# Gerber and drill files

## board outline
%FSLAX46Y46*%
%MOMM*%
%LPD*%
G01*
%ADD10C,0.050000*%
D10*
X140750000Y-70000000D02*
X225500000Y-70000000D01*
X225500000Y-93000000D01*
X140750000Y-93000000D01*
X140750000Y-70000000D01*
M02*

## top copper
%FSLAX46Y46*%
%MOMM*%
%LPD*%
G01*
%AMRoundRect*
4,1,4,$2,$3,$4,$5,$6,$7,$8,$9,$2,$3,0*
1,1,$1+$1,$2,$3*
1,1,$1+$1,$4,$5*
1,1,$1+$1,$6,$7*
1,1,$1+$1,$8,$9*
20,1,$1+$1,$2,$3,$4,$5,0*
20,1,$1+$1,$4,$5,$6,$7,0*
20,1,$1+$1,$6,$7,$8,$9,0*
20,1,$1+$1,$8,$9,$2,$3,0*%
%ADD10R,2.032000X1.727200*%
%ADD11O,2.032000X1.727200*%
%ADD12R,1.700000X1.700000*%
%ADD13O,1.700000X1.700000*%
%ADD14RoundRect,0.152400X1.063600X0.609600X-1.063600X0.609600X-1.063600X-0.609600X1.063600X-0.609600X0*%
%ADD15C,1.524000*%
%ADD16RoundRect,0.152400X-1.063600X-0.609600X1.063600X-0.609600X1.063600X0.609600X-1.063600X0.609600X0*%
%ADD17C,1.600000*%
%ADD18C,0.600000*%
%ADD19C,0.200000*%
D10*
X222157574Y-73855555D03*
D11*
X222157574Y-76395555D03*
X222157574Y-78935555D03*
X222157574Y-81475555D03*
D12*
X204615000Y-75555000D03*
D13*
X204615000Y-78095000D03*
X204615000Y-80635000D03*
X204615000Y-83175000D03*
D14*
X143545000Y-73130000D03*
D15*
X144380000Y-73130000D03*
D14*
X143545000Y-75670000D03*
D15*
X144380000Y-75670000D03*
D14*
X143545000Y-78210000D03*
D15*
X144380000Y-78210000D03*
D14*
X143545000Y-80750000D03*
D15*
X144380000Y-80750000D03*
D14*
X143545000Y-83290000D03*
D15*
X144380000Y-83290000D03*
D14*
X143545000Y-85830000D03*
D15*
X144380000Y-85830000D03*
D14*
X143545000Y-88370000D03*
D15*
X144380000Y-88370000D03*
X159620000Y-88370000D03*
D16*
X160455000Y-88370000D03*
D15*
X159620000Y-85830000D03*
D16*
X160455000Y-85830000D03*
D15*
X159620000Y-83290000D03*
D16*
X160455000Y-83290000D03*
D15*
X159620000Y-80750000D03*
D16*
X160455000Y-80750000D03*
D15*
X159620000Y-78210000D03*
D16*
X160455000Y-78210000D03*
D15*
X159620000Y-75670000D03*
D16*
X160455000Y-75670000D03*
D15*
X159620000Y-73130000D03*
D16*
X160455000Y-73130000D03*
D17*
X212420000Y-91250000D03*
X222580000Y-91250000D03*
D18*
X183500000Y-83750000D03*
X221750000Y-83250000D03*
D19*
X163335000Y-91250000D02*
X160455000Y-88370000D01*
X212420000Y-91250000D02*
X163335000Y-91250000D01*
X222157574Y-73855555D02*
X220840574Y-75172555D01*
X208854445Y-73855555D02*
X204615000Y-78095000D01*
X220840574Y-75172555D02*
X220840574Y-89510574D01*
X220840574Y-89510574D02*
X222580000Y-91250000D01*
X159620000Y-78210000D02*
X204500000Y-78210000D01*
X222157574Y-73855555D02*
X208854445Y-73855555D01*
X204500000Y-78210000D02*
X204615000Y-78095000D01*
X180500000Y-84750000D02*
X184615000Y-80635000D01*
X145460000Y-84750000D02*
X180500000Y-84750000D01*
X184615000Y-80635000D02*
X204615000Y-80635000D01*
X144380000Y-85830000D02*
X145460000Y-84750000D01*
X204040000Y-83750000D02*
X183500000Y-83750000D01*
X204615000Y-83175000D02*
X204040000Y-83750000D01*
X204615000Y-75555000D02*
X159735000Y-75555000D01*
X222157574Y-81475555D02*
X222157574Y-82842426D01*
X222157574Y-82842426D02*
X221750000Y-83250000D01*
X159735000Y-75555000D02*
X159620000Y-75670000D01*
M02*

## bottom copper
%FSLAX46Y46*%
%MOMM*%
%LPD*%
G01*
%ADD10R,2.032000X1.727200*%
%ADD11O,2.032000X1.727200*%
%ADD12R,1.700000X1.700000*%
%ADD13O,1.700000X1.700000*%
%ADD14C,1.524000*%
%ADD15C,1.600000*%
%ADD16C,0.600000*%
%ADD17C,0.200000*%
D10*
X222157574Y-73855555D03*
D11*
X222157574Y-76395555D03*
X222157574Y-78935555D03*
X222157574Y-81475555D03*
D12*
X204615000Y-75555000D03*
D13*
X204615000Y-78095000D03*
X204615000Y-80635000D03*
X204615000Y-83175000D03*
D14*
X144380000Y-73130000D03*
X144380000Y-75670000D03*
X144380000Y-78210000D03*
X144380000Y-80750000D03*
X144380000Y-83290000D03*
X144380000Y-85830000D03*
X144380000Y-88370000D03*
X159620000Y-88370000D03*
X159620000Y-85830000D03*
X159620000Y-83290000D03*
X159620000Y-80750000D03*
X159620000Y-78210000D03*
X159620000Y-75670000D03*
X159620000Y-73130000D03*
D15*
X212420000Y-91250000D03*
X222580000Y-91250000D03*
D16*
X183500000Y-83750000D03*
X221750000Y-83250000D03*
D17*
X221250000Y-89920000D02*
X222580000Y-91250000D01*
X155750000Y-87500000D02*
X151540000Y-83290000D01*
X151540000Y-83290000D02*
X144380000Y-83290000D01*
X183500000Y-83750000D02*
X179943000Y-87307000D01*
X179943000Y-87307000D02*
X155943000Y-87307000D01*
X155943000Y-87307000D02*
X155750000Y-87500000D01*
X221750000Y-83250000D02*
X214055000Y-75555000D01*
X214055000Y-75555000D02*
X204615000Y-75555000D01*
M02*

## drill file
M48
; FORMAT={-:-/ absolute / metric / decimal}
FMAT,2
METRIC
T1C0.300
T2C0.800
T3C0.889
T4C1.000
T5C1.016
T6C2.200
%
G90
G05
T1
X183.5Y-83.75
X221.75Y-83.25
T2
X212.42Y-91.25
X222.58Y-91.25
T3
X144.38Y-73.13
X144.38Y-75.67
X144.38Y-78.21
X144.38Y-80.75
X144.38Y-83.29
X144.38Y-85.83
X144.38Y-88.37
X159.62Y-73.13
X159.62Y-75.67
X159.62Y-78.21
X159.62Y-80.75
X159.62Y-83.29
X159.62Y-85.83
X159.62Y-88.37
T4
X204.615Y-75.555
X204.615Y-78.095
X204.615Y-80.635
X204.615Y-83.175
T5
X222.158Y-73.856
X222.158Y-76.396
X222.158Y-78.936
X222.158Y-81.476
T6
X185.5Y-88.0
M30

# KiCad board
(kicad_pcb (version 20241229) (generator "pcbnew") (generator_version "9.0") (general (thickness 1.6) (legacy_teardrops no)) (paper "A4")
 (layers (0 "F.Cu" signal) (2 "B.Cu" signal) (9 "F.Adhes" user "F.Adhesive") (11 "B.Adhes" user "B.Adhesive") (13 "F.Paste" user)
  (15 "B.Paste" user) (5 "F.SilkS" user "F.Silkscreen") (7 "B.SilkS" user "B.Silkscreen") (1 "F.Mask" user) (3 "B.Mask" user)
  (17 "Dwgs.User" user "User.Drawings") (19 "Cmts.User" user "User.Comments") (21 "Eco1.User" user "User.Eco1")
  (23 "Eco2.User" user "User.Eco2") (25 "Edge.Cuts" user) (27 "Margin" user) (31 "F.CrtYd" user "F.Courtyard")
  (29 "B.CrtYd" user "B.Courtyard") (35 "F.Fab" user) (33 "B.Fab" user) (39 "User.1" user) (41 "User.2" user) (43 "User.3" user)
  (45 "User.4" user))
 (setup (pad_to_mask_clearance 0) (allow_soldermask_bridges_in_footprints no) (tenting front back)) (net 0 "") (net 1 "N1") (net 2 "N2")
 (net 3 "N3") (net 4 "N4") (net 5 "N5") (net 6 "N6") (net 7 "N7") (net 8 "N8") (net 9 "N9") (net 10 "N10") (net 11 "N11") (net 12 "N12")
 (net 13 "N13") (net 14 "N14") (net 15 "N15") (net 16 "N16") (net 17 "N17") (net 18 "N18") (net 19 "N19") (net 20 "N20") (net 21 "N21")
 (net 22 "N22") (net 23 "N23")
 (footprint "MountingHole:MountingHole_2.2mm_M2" (layer "F.Cu") (at 185.5 88)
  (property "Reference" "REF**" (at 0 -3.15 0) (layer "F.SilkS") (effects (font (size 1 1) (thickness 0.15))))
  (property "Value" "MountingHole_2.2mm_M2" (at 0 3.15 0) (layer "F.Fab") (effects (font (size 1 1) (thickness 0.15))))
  (pad "" np_thru_hole circle (at 0 0) (size 2.2 2.2) (drill 2.2) (layers "*.Cu" "*.Mask")))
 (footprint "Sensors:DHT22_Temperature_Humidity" (layer "F.Cu") (at 222.157574 77.665555 -90)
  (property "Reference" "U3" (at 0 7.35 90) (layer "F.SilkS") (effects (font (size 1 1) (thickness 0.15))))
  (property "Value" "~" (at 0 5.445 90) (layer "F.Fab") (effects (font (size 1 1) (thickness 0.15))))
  (pad "1" thru_hole rect (at -3.81 0) (size 2.032 1.7272) (drill 1.016) (layers "*.Cu" "*.Mask" "F.SilkS") (remove_unused_layers no)
   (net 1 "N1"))
  (pad "2" thru_hole oval (at -1.27 0) (size 2.032 1.7272) (drill 1.016) (layers "*.Cu" "*.Mask" "F.SilkS") (remove_unused_layers no))
  (pad "3" thru_hole oval (at 1.27 0) (size 2.032 1.7272) (drill 1.016) (layers "*.Cu" "*.Mask" "F.SilkS") (remove_unused_layers no)
   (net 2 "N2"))
  (pad "4" thru_hole oval (at 3.81 0) (size 2.032 1.7272) (drill 1.016) (layers "*.Cu" "*.Mask" "F.SilkS") (remove_unused_layers no)
   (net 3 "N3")))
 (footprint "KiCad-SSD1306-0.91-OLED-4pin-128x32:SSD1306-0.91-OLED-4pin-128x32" (layer "F.Cu") (at 168.115 73.365)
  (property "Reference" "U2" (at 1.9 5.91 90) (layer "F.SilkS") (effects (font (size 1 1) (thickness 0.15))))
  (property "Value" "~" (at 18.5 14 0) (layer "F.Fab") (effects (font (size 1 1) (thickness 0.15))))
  (pad "1" thru_hole rect (at 36.5 2.19) (size 1.7 1.7) (drill 1) (layers "*.Cu" "*.Mask") (remove_unused_layers no) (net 3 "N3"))
  (pad "2" thru_hole oval (at 36.5 4.73) (size 1.7 1.7) (drill 1) (layers "*.Cu" "*.Mask") (remove_unused_layers no) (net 1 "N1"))
  (pad "3" thru_hole oval (at 36.5 7.27) (size 1.7 1.7) (drill 1) (layers "*.Cu" "*.Mask") (remove_unused_layers no) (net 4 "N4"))
  (pad "4" thru_hole oval (at 36.5 9.81) (size 1.7 1.7) (drill 1) (layers "*.Cu" "*.Mask") (remove_unused_layers no) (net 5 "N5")))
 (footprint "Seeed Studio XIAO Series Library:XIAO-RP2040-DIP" (layer "F.Cu") (at 152 80.75)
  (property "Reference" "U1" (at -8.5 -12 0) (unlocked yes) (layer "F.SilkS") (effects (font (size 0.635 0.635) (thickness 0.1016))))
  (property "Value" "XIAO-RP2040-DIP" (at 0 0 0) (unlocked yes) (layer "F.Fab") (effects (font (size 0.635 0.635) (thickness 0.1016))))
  (pad "1" smd roundrect (at -8.455 -7.62 180) (size 2.432 1.524) (layers "F.Cu" "F.Mask") (roundrect_rratio 0.1) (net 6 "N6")
   (thermal_bridge_angle 45))
  (pad "1" thru_hole circle (at -7.62 -7.62 180) (size 1.524 1.524) (drill 0.889) (layers "*.Cu" "*.Mask") (remove_unused_layers no)
   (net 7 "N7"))
  (pad "2" smd roundrect (at -8.455 -5.08 180) (size 2.432 1.524) (layers "F.Cu" "F.Mask") (roundrect_rratio 0.1) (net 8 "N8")
   (thermal_bridge_angle 45))
  (pad "2" thru_hole circle (at -7.62 -5.08 180) (size 1.524 1.524) (drill 0.889) (layers "*.Cu" "*.Mask") (remove_unused_layers no)
   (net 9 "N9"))
  (pad "3" smd roundrect (at -8.455 -2.54 180) (size 2.432 1.524) (layers "F.Cu" "F.Mask") (roundrect_rratio 0.1) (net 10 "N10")
   (thermal_bridge_angle 45))
  (pad "3" thru_hole circle (at -7.62 -2.54 180) (size 1.524 1.524) (drill 0.889) (layers "*.Cu" "*.Mask") (remove_unused_layers no)
   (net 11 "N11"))
  (pad "4" smd roundrect (at -8.455 0 180) (size 2.432 1.524) (layers "F.Cu" "F.Mask") (roundrect_rratio 0.1) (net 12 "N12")
   (thermal_bridge_angle 45))
  (pad "4" thru_hole circle (at -7.62 0 180) (size 1.524 1.524) (drill 0.889) (layers "*.Cu" "*.Mask") (remove_unused_layers no)
   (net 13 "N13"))
  (pad "5" smd roundrect (at -8.455 2.54 180) (size 2.432 1.524) (layers "F.Cu" "F.Mask") (roundrect_rratio 0.1) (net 5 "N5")
   (thermal_bridge_angle 45))
  (pad "5" thru_hole circle (at -7.62 2.54 180) (size 1.524 1.524) (drill 0.889) (layers "*.Cu" "*.Mask") (remove_unused_layers no)
   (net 5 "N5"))
  (pad "6" smd roundrect (at -8.455 5.08 180) (size 2.432 1.524) (layers "F.Cu" "F.Mask") (roundrect_rratio 0.1) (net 4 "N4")
   (thermal_bridge_angle 45))
  (pad "6" thru_hole circle (at -7.62 5.08 180) (size 1.524 1.524) (drill 0.889) (layers "*.Cu" "*.Mask") (remove_unused_layers no)
   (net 4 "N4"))
  (pad "7" smd roundrect (at -8.455 7.62 180) (size 2.432 1.524) (layers "F.Cu" "F.Mask") (roundrect_rratio 0.1) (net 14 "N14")
   (thermal_bridge_angle 45))
  (pad "7" thru_hole circle (at -7.62 7.62 180) (size 1.524 1.524) (drill 0.889) (layers "*.Cu" "*.Mask") (remove_unused_layers no)
   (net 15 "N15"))
  (pad "8" thru_hole circle (at 7.62 7.62) (size 1.524 1.524) (drill 0.889) (layers "*.Cu" "*.Mask") (remove_unused_layers no)
   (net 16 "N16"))
  (pad "8" smd roundrect (at 8.455 7.62) (size 2.432 1.524) (layers "F.Cu" "F.Mask") (roundrect_rratio 0.1) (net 16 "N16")
   (thermal_bridge_angle 45))
  (pad "9" thru_hole circle (at 7.62 5.08) (size 1.524 1.524) (drill 0.889) (layers "*.Cu" "*.Mask") (remove_unused_layers no)
   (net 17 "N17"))
  (pad "9" smd roundrect (at 8.455 5.08) (size 2.432 1.524) (layers "F.Cu" "F.Mask") (roundrect_rratio 0.1) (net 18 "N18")
   (thermal_bridge_angle 45))
  (pad "10" thru_hole circle (at 7.62 2.54) (size 1.524 1.524) (drill 0.889) (layers "*.Cu" "*.Mask") (remove_unused_layers no)
   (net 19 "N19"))
  (pad "10" smd roundrect (at 8.455 2.54) (size 2.432 1.524) (layers "F.Cu" "F.Mask") (roundrect_rratio 0.1) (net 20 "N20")
   (thermal_bridge_angle 45))
  (pad "11" thru_hole circle (at 7.62 0) (size 1.524 1.524) (drill 0.889) (layers "*.Cu" "*.Mask") (remove_unused_layers no) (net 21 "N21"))
  (pad "11" smd roundrect (at 8.455 0) (size 2.432 1.524) (layers "F.Cu" "F.Mask") (roundrect_rratio 0.1) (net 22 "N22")
   (thermal_bridge_angle 45))
  (pad "12" thru_hole circle (at 7.62 -2.54) (size 1.524 1.524) (drill 0.889) (layers "*.Cu" "*.Mask") (remove_unused_layers no)
   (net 1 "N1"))
  (pad "12" smd roundrect (at 8.455 -2.54) (size 2.432 1.524) (layers "F.Cu" "F.Mask") (roundrect_rratio 0.1) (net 1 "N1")
   (thermal_bridge_angle 45))
  (pad "13" thru_hole circle (at 7.62 -5.08) (size 1.524 1.524) (drill 0.889) (layers "*.Cu" "*.Mask") (remove_unused_layers no)
   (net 3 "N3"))
  (pad "13" smd roundrect (at 8.455 -5.08) (size 2.432 1.524) (layers "F.Cu" "F.Mask") (roundrect_rratio 0.1) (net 3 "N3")
   (thermal_bridge_angle 45))
  (pad "14" thru_hole circle (at 7.62 -7.62) (size 1.524 1.524) (drill 0.889) (layers "*.Cu" "*.Mask") (remove_unused_layers no)
   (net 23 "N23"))
  (pad "14" smd roundrect (at 8.455 -7.62) (size 2.432 1.524) (layers "F.Cu" "F.Mask") (roundrect_rratio 0.1) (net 23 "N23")
   (thermal_bridge_angle 45)))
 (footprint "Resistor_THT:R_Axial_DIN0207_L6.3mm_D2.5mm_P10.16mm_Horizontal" (layer "F.Cu") (at 212.42 91.25)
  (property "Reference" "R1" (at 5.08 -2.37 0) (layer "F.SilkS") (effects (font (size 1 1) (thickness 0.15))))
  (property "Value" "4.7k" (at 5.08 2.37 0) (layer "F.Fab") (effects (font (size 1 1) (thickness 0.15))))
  (pad "1" thru_hole circle (at 0 0) (size 1.6 1.6) (drill 0.8) (layers "*.Cu" "*.Mask") (remove_unused_layers no) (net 16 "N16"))
  (pad "2" thru_hole circle (at 10.16 0) (size 1.6 1.6) (drill 0.8) (layers "*.Cu" "*.Mask") (remove_unused_layers no) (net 1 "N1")))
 (gr_rect (start 140.75 70) (end 225.5 93) (stroke (width 0.05) (type default)) (fill no) (layer "Edge.Cuts"))
 (segment (start 163.335 91.25) (end 160.455 88.37) (width 0.2) (layer "F.Cu") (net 16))
 (segment (start 212.42 91.25) (end 163.335 91.25) (width 0.2) (layer "F.Cu") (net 16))
 (segment (start 222.157574 73.855555) (end 220.840574 75.172555) (width 0.2) (layer "F.Cu") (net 1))
 (segment (start 208.854445 73.855555) (end 204.615 78.095) (width 0.2) (layer "F.Cu") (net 1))
 (segment (start 220.840574 75.172555) (end 220.840574 89.510574) (width 0.2) (layer "F.Cu") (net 1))
 (segment (start 220.840574 89.510574) (end 222.58 91.25) (width 0.2) (layer "F.Cu") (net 1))
 (segment (start 159.62 78.21) (end 204.5 78.21) (width 0.2) (layer "F.Cu") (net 1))
 (segment (start 222.157574 73.855555) (end 208.854445 73.855555) (width 0.2) (layer "F.Cu") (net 1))
 (segment (start 204.5 78.21) (end 204.615 78.095) (width 0.2) (layer "F.Cu") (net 1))
 (segment (start 221.25 89.92) (end 222.58 91.25) (width 0.2) (layer "B.Cu") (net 1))
 (segment (start 180.5 84.75) (end 184.615 80.635) (width 0.2) (layer "F.Cu") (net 4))
 (segment (start 145.46 84.75) (end 180.5 84.75) (width 0.2) (layer "F.Cu") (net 4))
 (segment (start 184.615 80.635) (end 204.615 80.635) (width 0.2) (layer "F.Cu") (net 4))
 (segment (start 144.38 85.83) (end 145.46 84.75) (width 0.2) (layer "F.Cu") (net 4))
 (segment (start 204.04 83.75) (end 183.5 83.75) (width 0.2) (layer "F.Cu") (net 5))
 (segment (start 204.615 83.175) (end 204.04 83.75) (width 0.2) (layer "F.Cu") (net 5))
 (via (at 183.5 83.75) (size 0.6) (drill 0.3) (layers "F.Cu" "B.Cu") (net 5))
 (segment (start 155.75 87.5) (end 151.54 83.29) (width 0.2) (layer "B.Cu") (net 5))
 (segment (start 151.54 83.29) (end 144.38 83.29) (width 0.2) (layer "B.Cu") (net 5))
 (segment (start 183.5 83.75) (end 179.943 87.307) (width 0.2) (layer "B.Cu") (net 5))
 (segment (start 179.943 87.307) (end 155.943 87.307) (width 0.2) (layer "B.Cu") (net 5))
 (segment (start 155.943 87.307) (end 155.75 87.5) (width 0.2) (layer "B.Cu") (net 5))
 (segment (start 204.615 75.555) (end 159.735 75.555) (width 0.2) (layer "F.Cu") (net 3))
 (segment (start 222.157574 81.475555) (end 222.157574 82.842426) (width 0.2) (layer "F.Cu") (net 3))
 (segment (start 222.157574 82.842426) (end 221.75 83.25) (width 0.2) (layer "F.Cu") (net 3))
 (segment (start 159.735 75.555) (end 159.62 75.67) (width 0.2) (layer "F.Cu") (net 3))
 (via (at 221.75 83.25) (size 0.6) (drill 0.3) (layers "F.Cu" "B.Cu") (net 3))
 (segment (start 221.75 83.25) (end 214.055 75.555) (width 0.2) (layer "B.Cu") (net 3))
 (segment (start 214.055 75.555) (end 204.615 75.555) (width 0.2) (layer "B.Cu") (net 3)))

